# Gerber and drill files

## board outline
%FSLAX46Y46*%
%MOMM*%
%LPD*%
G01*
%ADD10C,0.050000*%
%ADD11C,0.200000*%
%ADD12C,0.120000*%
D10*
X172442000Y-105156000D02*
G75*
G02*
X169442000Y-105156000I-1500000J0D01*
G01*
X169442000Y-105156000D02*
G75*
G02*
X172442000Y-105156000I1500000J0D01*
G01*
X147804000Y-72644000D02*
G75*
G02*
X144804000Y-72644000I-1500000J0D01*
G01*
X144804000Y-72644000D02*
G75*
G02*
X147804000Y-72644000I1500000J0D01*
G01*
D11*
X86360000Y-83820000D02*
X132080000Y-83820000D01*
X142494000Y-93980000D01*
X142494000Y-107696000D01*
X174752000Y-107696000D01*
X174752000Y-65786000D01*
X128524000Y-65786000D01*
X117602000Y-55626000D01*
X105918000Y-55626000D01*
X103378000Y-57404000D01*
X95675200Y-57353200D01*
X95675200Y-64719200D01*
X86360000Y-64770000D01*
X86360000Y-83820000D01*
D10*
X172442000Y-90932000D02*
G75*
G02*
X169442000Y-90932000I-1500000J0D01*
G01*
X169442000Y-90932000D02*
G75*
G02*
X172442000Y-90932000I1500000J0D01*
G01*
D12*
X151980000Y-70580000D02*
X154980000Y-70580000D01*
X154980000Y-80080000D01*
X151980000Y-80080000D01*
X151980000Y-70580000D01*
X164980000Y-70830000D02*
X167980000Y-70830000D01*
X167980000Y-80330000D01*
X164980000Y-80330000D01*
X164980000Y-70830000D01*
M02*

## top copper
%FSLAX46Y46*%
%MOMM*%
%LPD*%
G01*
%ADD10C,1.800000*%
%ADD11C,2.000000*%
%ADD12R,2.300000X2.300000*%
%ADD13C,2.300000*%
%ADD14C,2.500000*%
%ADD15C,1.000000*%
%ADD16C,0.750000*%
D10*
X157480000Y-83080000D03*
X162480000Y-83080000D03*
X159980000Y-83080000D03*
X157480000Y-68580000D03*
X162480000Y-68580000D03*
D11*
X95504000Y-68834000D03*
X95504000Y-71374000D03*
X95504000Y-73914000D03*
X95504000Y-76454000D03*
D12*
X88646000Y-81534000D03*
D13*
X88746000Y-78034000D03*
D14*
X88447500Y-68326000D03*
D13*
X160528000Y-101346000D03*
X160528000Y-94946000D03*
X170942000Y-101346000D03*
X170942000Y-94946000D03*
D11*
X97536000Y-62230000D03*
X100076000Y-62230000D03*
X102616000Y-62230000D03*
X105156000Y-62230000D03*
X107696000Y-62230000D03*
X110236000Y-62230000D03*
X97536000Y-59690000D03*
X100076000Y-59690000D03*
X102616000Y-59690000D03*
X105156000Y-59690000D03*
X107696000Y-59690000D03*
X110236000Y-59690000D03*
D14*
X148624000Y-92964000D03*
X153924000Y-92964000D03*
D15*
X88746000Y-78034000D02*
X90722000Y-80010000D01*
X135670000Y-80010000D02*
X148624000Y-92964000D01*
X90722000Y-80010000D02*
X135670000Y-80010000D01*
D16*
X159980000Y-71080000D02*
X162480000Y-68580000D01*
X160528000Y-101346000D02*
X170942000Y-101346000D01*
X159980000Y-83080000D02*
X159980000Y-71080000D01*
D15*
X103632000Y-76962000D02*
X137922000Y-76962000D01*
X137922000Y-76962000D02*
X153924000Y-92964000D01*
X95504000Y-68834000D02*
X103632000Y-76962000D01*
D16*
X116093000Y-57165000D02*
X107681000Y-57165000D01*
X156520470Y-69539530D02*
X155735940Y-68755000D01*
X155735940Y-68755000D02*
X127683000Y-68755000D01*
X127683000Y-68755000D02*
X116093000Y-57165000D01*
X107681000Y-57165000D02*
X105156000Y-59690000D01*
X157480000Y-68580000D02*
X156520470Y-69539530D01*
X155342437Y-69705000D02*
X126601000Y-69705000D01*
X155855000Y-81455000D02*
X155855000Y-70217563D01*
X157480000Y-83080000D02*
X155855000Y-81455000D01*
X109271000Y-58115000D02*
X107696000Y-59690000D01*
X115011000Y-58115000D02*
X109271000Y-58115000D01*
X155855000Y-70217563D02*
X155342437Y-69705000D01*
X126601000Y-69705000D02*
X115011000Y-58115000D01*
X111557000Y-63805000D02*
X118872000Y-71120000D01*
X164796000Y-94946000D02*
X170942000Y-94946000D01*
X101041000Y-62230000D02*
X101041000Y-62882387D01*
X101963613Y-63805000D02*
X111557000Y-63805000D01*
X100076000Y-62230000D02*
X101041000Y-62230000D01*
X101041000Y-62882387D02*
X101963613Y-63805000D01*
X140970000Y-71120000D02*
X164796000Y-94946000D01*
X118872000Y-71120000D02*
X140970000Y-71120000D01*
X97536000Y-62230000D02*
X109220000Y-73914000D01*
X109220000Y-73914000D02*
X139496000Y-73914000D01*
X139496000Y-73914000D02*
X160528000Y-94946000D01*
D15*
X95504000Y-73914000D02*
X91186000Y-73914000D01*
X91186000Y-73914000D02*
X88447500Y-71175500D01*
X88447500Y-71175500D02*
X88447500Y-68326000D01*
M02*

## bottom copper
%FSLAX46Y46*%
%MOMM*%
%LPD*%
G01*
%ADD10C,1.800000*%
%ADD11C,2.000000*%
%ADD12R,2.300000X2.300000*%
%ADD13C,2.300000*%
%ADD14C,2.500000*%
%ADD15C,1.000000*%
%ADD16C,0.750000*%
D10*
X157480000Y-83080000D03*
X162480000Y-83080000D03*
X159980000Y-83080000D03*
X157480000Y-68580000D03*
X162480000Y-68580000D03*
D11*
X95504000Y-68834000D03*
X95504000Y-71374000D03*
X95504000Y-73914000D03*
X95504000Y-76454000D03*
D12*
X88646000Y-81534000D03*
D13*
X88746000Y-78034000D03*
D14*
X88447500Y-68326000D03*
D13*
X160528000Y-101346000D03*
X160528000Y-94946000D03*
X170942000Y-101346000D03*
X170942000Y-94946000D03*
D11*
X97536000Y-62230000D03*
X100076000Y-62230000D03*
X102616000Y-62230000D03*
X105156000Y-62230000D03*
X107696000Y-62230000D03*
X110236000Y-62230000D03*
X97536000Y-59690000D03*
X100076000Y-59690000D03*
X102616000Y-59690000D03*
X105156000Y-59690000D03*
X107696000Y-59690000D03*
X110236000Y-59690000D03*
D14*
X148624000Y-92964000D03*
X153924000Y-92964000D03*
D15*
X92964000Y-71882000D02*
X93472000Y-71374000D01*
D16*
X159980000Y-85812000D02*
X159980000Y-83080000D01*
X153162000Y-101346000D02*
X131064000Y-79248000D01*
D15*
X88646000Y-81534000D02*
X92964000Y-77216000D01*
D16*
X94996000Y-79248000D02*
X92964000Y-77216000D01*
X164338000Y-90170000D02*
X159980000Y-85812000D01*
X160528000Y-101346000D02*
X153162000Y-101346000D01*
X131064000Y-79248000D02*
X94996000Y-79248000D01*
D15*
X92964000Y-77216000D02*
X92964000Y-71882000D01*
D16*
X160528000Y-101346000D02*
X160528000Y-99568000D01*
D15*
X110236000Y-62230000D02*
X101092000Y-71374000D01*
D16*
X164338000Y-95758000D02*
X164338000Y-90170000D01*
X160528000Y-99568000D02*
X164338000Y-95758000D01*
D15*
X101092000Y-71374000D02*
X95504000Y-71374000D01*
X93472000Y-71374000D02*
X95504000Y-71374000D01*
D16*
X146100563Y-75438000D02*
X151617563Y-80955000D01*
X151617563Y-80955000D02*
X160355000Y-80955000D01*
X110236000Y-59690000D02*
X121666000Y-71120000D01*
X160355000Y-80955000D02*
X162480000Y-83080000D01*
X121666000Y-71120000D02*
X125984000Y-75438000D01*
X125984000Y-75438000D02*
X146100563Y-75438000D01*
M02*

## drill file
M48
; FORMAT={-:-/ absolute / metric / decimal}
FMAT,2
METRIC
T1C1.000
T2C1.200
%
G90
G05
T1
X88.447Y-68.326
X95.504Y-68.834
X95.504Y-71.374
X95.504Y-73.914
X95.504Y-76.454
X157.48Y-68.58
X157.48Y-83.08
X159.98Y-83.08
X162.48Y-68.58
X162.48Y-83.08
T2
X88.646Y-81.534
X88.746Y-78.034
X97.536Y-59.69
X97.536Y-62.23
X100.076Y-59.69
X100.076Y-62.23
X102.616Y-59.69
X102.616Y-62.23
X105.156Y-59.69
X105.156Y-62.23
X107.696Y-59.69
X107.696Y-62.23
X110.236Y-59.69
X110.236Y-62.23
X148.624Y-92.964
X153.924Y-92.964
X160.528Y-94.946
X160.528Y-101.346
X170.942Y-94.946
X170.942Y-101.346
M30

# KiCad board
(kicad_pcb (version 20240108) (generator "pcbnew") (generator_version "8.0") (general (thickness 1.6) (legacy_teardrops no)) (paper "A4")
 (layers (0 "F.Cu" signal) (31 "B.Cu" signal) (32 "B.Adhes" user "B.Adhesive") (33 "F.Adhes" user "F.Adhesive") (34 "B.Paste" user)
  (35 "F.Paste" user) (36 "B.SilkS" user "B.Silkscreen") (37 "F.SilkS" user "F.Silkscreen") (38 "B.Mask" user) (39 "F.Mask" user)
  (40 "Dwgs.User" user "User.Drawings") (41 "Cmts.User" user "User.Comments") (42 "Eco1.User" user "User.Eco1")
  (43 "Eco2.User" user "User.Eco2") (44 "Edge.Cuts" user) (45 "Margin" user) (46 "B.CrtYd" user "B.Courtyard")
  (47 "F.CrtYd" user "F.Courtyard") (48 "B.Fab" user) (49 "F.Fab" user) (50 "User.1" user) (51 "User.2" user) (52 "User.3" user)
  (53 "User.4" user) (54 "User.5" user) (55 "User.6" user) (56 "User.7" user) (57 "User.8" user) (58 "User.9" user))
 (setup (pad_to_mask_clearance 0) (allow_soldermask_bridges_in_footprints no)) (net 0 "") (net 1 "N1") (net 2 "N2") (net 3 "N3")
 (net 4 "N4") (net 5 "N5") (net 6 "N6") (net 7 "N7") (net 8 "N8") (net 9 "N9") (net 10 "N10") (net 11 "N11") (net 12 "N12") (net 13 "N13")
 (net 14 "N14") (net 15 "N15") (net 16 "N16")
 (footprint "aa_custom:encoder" (layer "F.Cu") (at 169.48 80.08 90)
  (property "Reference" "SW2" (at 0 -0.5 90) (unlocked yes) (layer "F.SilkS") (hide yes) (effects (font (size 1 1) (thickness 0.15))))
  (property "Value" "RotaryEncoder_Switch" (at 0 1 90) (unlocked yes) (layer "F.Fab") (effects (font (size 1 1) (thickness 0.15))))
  (fp_rect (start 0 -17.5) (end 9.5 -14.5) (stroke (width 0.12) (type default)) (fill none) (layer "Edge.Cuts"))
  (fp_rect (start -0.25 -4.5) (end 9.25 -1.5) (stroke (width 0.12) (type default)) (fill none) (layer "Edge.Cuts"))
  (pad "A" thru_hole circle (at -3 -12 90) (size 1.8 1.8) (drill 1) (layers "*.Cu" "*.Mask") (remove_unused_layers no) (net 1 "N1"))
  (pad "B" thru_hole circle (at -3 -7 90) (size 1.8 1.8) (drill 1) (layers "*.Cu" "*.Mask") (remove_unused_layers no) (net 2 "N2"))
  (pad "C" thru_hole circle (at -3 -9.5 90) (size 1.8 1.8) (drill 1) (layers "*.Cu" "*.Mask") (remove_unused_layers no) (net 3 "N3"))
  (pad "S1" thru_hole circle (at 11.5 -12 90) (size 1.8 1.8) (drill 1) (layers "*.Cu" "*.Mask") (remove_unused_layers no) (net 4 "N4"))
  (pad "S2" thru_hole circle (at 11.5 -7 90) (size 1.8 1.8) (drill 1) (layers "*.Cu" "*.Mask") (remove_unused_layers no) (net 3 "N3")))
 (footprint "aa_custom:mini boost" (layer "F.Cu") (at 95.504 79.629)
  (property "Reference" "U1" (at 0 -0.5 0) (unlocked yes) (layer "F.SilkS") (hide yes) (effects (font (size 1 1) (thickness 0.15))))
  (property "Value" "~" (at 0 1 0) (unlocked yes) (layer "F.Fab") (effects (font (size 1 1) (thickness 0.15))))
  (pad "1" thru_hole circle (at 0 -10.795) (size 2 2) (drill 1) (layers "*.Cu" "*.Mask") (remove_unused_layers no) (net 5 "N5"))
  (pad "2" thru_hole circle (at 0 -8.255) (size 2 2) (drill 1) (layers "*.Cu" "*.Mask") (remove_unused_layers no) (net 3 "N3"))
  (pad "3" thru_hole circle (at 0 -5.715) (size 2 2) (drill 1) (layers "*.Cu" "*.Mask") (remove_unused_layers no) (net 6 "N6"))
  (pad "4" thru_hole circle (at 0 -3.175) (size 2 2) (drill 1) (layers "*.Cu" "*.Mask") (remove_unused_layers no) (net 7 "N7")))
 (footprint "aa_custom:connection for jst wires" (layer "F.Cu") (at 92.946 79.334 90)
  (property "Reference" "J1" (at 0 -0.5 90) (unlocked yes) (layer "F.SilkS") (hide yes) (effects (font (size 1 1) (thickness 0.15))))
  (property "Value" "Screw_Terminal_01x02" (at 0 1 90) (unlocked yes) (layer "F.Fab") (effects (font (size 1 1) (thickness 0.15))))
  (pad "1" thru_hole rect (at -2.2 -4.3 90) (size 2.3 2.3) (drill 1.2) (layers "*.Cu" "*.Mask") (remove_unused_layers no) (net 3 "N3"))
  (pad "2" thru_hole circle (at 1.3 -4.2 90) (size 2.3 2.3) (drill 1.2) (layers "*.Cu" "*.Mask") (remove_unused_layers no) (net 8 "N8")))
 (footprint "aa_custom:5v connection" (layer "F.Cu") (at 92.8925 68.326 90)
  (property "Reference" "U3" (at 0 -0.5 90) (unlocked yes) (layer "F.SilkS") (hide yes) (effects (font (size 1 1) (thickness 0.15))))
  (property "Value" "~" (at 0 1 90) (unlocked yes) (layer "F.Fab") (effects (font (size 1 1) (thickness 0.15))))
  (pad "1" thru_hole circle (at 0 -4.445 90) (size 2.5 2.5) (drill 1) (layers "*.Cu" "*.Mask") (remove_unused_layers no) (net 6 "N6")))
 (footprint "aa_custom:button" (layer "F.Cu") (at 163.328 98.446 90)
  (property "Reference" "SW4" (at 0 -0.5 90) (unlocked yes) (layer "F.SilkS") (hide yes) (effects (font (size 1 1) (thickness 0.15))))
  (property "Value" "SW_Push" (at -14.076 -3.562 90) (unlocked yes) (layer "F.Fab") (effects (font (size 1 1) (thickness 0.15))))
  (pad "1" thru_hole circle (at -2.9 -2.8 90) (size 2.3 2.3) (drill 1.2) (layers "*.Cu" "*.Mask") (remove_unused_layers no) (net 3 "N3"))
  (pad "2" thru_hole circle (at 3.5 -2.8 90) (size 2.3 2.3) (drill 1.2) (layers "*.Cu" "*.Mask") (remove_unused_layers no) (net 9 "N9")))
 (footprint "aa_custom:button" (layer "F.Cu") (at 173.742 98.446 90)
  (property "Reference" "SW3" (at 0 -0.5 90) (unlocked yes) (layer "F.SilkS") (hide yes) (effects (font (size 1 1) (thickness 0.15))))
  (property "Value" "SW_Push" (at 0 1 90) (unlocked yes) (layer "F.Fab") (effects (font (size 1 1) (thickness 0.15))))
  (pad "1" thru_hole circle (at -2.9 -2.8 90) (size 2.3 2.3) (drill 1.2) (layers "*.Cu" "*.Mask") (remove_unused_layers no) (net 3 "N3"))
  (pad "2" thru_hole circle (at 3.5 -2.8 90) (size 2.3 2.3) (drill 1.2) (layers "*.Cu" "*.Mask") (remove_unused_layers no) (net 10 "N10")))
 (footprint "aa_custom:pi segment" (layer "F.Cu") (at 107.696 69.85 90)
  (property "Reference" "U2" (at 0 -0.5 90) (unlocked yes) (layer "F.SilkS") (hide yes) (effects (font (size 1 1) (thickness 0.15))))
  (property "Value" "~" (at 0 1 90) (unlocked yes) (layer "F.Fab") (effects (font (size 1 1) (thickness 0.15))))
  (pad "2" thru_hole circle (at 7.62 -10.16 90) (size 2 2) (drill 1.2) (layers "*.Cu" "*.Mask") (remove_unused_layers no) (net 9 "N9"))
  (pad "3" thru_hole circle (at 7.62 -7.62 90) (size 2 2) (drill 1.2) (layers "*.Cu" "*.Mask") (remove_unused_layers no) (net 10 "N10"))
  (pad "4" thru_hole circle (at 7.62 -5.08 90) (size 2 2) (drill 1.2) (layers "*.Cu" "*.Mask") (remove_unused_layers no) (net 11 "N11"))
  (pad "5" thru_hole circle (at 7.62 -2.54 90) (size 2 2) (drill 1.2) (layers "*.Cu" "*.Mask") (remove_unused_layers no) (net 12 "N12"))
  (pad "6" thru_hole circle (at 7.62 0 90) (size 2 2) (drill 1.2) (layers "*.Cu" "*.Mask") (remove_unused_layers no) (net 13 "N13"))
  (pad "7" thru_hole circle (at 7.62 2.54 90) (size 2 2) (drill 1.2) (layers "*.Cu" "*.Mask") (remove_unused_layers no) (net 3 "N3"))
  (pad "9" thru_hole circle (at 10.16 -10.16 90) (size 2 2) (drill 1.2) (layers "*.Cu" "*.Mask") (remove_unused_layers no) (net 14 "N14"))
  (pad "10" thru_hole circle (at 10.16 -7.62 90) (size 2 2) (drill 1.2) (layers "*.Cu" "*.Mask") (remove_unused_layers no) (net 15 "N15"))
  (pad "11" thru_hole circle (at 10.16 -5.08 90) (size 2 2) (drill 1.2) (layers "*.Cu" "*.Mask") (remove_unused_layers no) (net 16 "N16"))
  (pad "12" thru_hole circle (at 10.16 -2.54 90) (size 2 2) (drill 1.2) (layers "*.Cu" "*.Mask") (remove_unused_layers no) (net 4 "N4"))
  (pad "13" thru_hole circle (at 10.16 0 90) (size 2 2) (drill 1.2) (layers "*.Cu" "*.Mask") (remove_unused_layers no) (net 1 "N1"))
  (pad "14" thru_hole circle (at 10.16 2.54 90) (size 2 2) (drill 1.2) (layers "*.Cu" "*.Mask") (remove_unused_layers no) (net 2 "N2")))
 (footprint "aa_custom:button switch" (layer "F.Cu") (at 152.524 101.964)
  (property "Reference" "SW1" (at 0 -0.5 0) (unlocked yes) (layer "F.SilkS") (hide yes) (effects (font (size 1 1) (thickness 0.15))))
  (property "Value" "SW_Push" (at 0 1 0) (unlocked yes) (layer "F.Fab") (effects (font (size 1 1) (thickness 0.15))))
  (pad "1" thru_hole circle (at -3.9 -9) (size 2.5 2.5) (drill 1.2) (layers "*.Cu" "*.Mask") (remove_unused_layers no) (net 8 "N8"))
  (pad "2" thru_hole circle (at 1.4 -9) (size 2.5 2.5) (drill 1.2) (layers "*.Cu" "*.Mask") (remove_unused_layers no) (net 5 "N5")))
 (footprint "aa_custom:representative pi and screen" (layer "F.Cu") (at 68.326 69.596)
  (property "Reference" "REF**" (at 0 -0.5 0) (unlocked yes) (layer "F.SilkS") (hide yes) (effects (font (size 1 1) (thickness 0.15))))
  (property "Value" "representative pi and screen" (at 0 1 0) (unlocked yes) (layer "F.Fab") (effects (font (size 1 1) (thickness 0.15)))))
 (gr_circle (center 170.942 105.156) (end 172.442 105.156) (stroke (width 0.05) (type default)) (fill none) (layer "Edge.Cuts"))
 (gr_circle (center 146.304 72.644) (end 147.804 72.644) (stroke (width 0.05) (type default)) (fill none) (layer "Edge.Cuts"))
 (gr_poly
  (pts (xy 86.36 83.82) (xy 132.08 83.82) (xy 142.494 93.98) (xy 142.494 107.696) (xy 174.752 107.696) (xy 174.752 65.786)
   (xy 128.524 65.786) (xy 117.602 55.626) (xy 105.918 55.626) (xy 103.378 57.404) (xy 95.6752 57.3532) (xy 95.6752 64.7192)
   (xy 86.36 64.77))
  (stroke (width 0.2) (type solid)) (fill none) (layer "Edge.Cuts"))
 (gr_circle (center 170.942 90.932) (end 172.442 90.932) (stroke (width 0.05) (type default)) (fill none) (layer "Edge.Cuts"))
 (segment (start 88.746 78.034) (end 90.722 80.01) (width 1) (layer "F.Cu") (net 8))
 (segment (start 135.67 80.01) (end 148.624 92.964) (width 1) (layer "F.Cu") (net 8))
 (segment (start 90.722 80.01) (end 135.67 80.01) (width 1) (layer "F.Cu") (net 8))
 (segment (start 159.98 71.08) (end 162.48 68.58) (width 0.75) (layer "F.Cu") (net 3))
 (segment (start 160.528 101.346) (end 170.942 101.346) (width 0.75) (layer "F.Cu") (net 3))
 (segment (start 159.98 83.08) (end 159.98 71.08) (width 0.75) (layer "F.Cu") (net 3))
 (segment (start 92.964 71.882) (end 93.472 71.374) (width 1) (layer "B.Cu") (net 3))
 (segment (start 159.98 85.812) (end 159.98 83.08) (width 0.75) (layer "B.Cu") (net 3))
 (segment (start 153.162 101.346) (end 131.064 79.248) (width 0.75) (layer "B.Cu") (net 3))
 (segment (start 88.646 81.534) (end 92.964 77.216) (width 1) (layer "B.Cu") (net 3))
 (segment (start 94.996 79.248) (end 92.964 77.216) (width 0.75) (layer "B.Cu") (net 3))
 (segment (start 164.338 90.17) (end 159.98 85.812) (width 0.75) (layer "B.Cu") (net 3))
 (segment (start 160.528 101.346) (end 153.162 101.346) (width 0.75) (layer "B.Cu") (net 3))
 (segment (start 131.064 79.248) (end 94.996 79.248) (width 0.75) (layer "B.Cu") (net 3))
 (segment (start 92.964 77.216) (end 92.964 71.882) (width 1) (layer "B.Cu") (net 3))
 (segment (start 160.528 101.346) (end 160.528 99.568) (width 0.75) (layer "B.Cu") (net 3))
 (segment (start 110.236 62.23) (end 101.092 71.374) (width 1) (layer "B.Cu") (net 3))
 (segment (start 164.338 95.758) (end 164.338 90.17) (width 0.75) (layer "B.Cu") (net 3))
 (segment (start 160.528 99.568) (end 164.338 95.758) (width 0.75) (layer "B.Cu") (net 3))
 (segment (start 101.092 71.374) (end 95.504 71.374) (width 1) (layer "B.Cu") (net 3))
 (segment (start 93.472 71.374) (end 95.504 71.374) (width 1) (layer "B.Cu") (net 3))
 (segment (start 103.632 76.962) (end 137.922 76.962) (width 1) (layer "F.Cu") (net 5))
 (segment (start 137.922 76.962) (end 153.924 92.964) (width 1) (layer "F.Cu") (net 5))
 (segment (start 95.504 68.834) (end 103.632 76.962) (width 1) (layer "F.Cu") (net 5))
 (segment (start 116.093 57.165) (end 107.681 57.165) (width 0.75) (layer "F.Cu") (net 4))
 (segment (start 156.52047 69.53953) (end 155.73594 68.755) (width 0.75) (layer "F.Cu") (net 4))
 (segment (start 155.73594 68.755) (end 127.683 68.755) (width 0.75) (layer "F.Cu") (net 4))
 (segment (start 127.683 68.755) (end 116.093 57.165) (width 0.75) (layer "F.Cu") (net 4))
 (segment (start 107.681 57.165) (end 105.156 59.69) (width 0.75) (layer "F.Cu") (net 4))
 (segment (start 157.48 68.58) (end 156.52047 69.53953) (width 0.75) (layer "F.Cu") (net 4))
 (segment (start 146.100563 75.438) (end 151.617563 80.955) (width 0.75) (layer "B.Cu") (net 2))
 (segment (start 151.617563 80.955) (end 160.355 80.955) (width 0.75) (layer "B.Cu") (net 2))
 (segment (start 110.236 59.69) (end 121.666 71.12) (width 0.75) (layer "B.Cu") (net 2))
 (segment (start 160.355 80.955) (end 162.48 83.08) (width 0.75) (layer "B.Cu") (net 2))
 (segment (start 121.666 71.12) (end 125.984 75.438) (width 0.75) (layer "B.Cu") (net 2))
 (segment (start 125.984 75.438) (end 146.100563 75.438) (width 0.75) (layer "B.Cu") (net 2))
 (segment (start 155.342437 69.705) (end 126.601 69.705) (width 0.75) (layer "F.Cu") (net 1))
 (segment (start 155.855 81.455) (end 155.855 70.217563) (width 0.75) (layer "F.Cu") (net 1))
 (segment (start 157.48 83.08) (end 155.855 81.455) (width 0.75) (layer "F.Cu") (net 1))
 (segment (start 109.271 58.115) (end 107.696 59.69) (width 0.75) (layer "F.Cu") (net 1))
 (segment (start 115.011 58.115) (end 109.271 58.115) (width 0.75) (layer "F.Cu") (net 1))
 (segment (start 155.855 70.217563) (end 155.342437 69.705) (width 0.75) (layer "F.Cu") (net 1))
 (segment (start 126.601 69.705) (end 115.011 58.115) (width 0.75) (layer "F.Cu") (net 1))
 (segment (start 111.557 63.805) (end 118.872 71.12) (width 0.75) (layer "F.Cu") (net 10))
 (segment (start 164.796 94.946) (end 170.942 94.946) (width 0.75) (layer "F.Cu") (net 10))
 (segment (start 101.041 62.23) (end 101.041 62.882387) (width 0.75) (layer "F.Cu") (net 10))
 (segment (start 101.963613 63.805) (end 111.557 63.805) (width 0.75) (layer "F.Cu") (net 10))
 (segment (start 100.076 62.23) (end 101.041 62.23) (width 0.75) (layer "F.Cu") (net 10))
 (segment (start 101.041 62.882387) (end 101.963613 63.805) (width 0.75) (layer "F.Cu") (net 10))
 (segment (start 140.97 71.12) (end 164.796 94.946) (width 0.75) (layer "F.Cu") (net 10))
 (segment (start 118.872 71.12) (end 140.97 71.12) (width 0.75) (layer "F.Cu") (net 10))
 (segment (start 97.536 62.23) (end 109.22 73.914) (width 0.75) (layer "F.Cu") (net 9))
 (segment (start 109.22 73.914) (end 139.496 73.914) (width 0.75) (layer "F.Cu") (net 9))
 (segment (start 139.496 73.914) (end 160.528 94.946) (width 0.75) (layer "F.Cu") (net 9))
 (segment (start 95.504 73.914) (end 91.186 73.914) (width 1) (layer "F.Cu") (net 6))
 (segment (start 91.186 73.914) (end 88.4475 71.1755) (width 1) (layer "F.Cu") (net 6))
 (segment (start 88.4475 71.1755) (end 88.4475 68.326) (width 1) (layer "F.Cu") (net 6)))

